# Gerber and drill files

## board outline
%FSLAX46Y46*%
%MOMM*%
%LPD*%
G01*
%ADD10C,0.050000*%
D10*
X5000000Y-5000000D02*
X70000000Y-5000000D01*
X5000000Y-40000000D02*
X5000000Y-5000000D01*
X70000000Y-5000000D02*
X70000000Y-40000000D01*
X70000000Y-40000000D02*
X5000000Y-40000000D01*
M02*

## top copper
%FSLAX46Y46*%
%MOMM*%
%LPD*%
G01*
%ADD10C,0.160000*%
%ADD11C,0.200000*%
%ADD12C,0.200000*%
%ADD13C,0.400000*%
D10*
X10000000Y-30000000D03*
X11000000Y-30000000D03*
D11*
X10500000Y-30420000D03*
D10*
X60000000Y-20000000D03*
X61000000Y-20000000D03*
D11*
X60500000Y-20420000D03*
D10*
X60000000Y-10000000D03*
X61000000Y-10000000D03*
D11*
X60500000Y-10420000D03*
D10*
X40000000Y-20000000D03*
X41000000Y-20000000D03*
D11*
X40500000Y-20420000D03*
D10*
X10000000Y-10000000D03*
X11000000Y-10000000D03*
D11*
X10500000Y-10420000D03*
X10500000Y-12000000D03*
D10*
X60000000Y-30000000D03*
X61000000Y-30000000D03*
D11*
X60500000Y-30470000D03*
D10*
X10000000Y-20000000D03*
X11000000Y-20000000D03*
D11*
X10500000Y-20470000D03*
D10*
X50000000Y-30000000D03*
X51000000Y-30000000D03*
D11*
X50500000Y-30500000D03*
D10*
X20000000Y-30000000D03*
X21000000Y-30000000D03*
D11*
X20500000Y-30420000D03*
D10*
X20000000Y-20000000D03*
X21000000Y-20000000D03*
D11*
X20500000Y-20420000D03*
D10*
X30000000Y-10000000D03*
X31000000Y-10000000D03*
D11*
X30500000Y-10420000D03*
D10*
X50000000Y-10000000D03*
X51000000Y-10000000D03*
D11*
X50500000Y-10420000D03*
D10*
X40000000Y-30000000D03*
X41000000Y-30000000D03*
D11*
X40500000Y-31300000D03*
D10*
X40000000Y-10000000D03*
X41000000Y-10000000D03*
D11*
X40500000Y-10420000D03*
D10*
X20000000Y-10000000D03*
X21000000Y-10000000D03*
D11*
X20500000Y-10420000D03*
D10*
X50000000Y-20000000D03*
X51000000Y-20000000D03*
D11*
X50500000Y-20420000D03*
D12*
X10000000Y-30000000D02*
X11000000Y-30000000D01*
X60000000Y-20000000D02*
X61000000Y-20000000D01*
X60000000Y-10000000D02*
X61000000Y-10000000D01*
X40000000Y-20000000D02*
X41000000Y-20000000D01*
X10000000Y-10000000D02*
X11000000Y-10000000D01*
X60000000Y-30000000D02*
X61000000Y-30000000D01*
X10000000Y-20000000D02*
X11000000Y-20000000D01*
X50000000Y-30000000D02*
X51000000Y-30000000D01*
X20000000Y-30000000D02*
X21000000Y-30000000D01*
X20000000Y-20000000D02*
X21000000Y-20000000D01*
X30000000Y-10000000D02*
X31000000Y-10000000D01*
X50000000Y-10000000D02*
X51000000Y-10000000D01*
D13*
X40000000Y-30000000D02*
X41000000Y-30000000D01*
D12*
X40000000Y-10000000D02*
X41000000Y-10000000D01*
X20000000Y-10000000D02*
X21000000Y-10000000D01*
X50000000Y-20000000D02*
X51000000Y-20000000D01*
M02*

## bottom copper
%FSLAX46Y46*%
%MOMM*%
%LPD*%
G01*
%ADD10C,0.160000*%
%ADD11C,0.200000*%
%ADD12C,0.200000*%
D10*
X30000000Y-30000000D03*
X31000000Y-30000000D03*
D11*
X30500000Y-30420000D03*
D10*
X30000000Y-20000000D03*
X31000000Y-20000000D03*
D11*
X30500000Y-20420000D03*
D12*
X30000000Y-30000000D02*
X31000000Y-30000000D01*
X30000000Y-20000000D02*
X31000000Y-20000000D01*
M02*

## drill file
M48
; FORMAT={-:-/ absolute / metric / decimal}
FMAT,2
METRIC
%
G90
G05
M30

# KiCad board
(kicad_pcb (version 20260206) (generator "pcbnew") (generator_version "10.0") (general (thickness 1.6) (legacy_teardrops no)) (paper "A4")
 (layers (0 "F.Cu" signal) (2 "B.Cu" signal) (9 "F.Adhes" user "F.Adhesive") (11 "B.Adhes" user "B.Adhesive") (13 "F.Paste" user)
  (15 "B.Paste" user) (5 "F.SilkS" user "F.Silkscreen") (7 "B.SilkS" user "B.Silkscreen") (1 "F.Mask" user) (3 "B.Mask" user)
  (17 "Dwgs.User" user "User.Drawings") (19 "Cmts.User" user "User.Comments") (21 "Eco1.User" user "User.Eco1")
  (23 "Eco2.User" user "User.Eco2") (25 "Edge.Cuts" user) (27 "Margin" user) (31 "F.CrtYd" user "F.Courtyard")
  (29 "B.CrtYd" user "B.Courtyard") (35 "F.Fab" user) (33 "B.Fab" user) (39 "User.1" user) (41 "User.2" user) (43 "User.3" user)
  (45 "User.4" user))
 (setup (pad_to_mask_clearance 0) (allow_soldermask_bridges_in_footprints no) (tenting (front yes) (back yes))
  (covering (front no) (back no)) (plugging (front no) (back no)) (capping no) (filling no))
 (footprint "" (layer "F.Cu") (at 10 30)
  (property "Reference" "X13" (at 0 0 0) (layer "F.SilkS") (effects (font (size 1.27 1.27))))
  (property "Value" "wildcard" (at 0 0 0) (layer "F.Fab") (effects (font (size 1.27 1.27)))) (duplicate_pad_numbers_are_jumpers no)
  (pad "1" smd circle (at 0 0) (size 0.16 0.16) (layers "F.Cu") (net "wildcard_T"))
  (pad "2" smd circle (at 1 0) (size 0.16 0.16) (layers "F.Cu") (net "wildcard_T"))
  (pad "3" smd circle (at 0.5 0.42) (size 0.2 0.2) (layers "F.Cu") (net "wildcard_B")))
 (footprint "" (layer "F.Cu") (at 60 20)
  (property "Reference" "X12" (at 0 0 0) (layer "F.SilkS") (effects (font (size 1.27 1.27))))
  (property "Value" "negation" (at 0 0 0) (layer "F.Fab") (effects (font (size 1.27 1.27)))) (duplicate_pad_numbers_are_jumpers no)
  (pad "1" smd circle (at 0 0) (size 0.16 0.16) (layers "F.Cu") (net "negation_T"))
  (pad "2" smd circle (at 1 0) (size 0.16 0.16) (layers "F.Cu") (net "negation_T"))
  (pad "3" smd circle (at 0.5 0.42) (size 0.2 0.2) (layers "F.Cu") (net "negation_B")))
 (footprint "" (layer "F.Cu") (at 60 10)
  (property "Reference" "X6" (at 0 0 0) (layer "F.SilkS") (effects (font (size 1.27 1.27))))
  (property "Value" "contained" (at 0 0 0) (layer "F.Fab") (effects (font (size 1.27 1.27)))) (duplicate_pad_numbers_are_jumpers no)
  (pad "1" smd circle (at 0 0) (size 0.16 0.16) (layers "F.Cu") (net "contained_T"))
  (pad "2" smd circle (at 1 0) (size 0.16 0.16) (layers "F.Cu") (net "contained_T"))
  (pad "3" smd circle (at 0.5 0.42) (size 0.2 0.2) (layers "F.Cu") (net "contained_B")))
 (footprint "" (layer "F.Cu") (at 40 20)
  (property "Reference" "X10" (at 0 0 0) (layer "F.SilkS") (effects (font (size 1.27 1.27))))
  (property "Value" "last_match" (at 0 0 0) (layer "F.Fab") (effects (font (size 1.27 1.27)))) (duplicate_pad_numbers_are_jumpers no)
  (pad "1" smd circle (at 0 0) (size 0.16 0.16) (layers "F.Cu") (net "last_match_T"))
  (pad "2" smd circle (at 1 0) (size 0.16 0.16) (layers "F.Cu") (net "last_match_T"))
  (pad "3" smd circle (at 0.5 0.42) (size 0.2 0.2) (layers "F.Cu") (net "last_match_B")))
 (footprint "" (layer "F.Cu") (at 10 10)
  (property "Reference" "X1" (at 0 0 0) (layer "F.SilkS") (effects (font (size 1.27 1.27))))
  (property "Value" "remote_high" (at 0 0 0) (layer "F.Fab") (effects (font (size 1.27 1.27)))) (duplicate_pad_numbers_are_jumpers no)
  (pad "1" smd circle (at 0 0) (size 0.16 0.16) (layers "F.Cu") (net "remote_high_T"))
  (pad "2" smd circle (at 1 0) (size 0.16 0.16) (layers "F.Cu") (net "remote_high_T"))
  (pad "3" smd circle (at 0.5 0.42) (size 0.2 0.2) (layers "F.Cu") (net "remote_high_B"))
  (pad "4" smd circle (at 0.5 2) (size 0.2 0.2) (layers "F.Cu") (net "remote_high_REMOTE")))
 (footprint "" (layer "F.Cu") (at 60 30)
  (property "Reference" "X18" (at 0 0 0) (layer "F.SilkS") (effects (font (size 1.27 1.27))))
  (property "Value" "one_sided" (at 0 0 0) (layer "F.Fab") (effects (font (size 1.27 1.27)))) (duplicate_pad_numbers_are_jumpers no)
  (pad "1" smd circle (at 0 0) (size 0.16 0.16) (layers "F.Cu") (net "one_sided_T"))
  (pad "2" smd circle (at 1 0) (size 0.16 0.16) (layers "F.Cu") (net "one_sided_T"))
  (pad "3" smd circle (at 0.5 0.47) (size 0.2 0.2) (layers "F.Cu") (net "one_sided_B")))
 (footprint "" (layer "F.Cu") (at 10 20)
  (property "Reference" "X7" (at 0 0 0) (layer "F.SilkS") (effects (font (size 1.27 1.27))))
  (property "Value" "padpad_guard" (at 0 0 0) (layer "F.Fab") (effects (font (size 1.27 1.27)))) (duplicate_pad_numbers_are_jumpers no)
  (pad "1" smd circle (at 0 0) (size 0.16 0.16) (layers "F.Cu") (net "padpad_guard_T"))
  (pad "2" smd circle (at 1 0) (size 0.16 0.16) (layers "F.Cu") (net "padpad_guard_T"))
  (pad "3" smd circle (at 0.5 0.47) (size 0.2 0.2) (layers "F.Cu") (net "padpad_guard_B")))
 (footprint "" (layer "F.Cu") (at 50 30)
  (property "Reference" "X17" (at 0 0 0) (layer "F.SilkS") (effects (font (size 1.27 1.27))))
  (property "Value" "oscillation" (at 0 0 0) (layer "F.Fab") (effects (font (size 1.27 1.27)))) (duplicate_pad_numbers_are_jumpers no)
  (pad "1" smd circle (at 0 0) (size 0.16 0.16) (layers "F.Cu") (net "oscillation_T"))
  (pad "2" smd circle (at 1 0) (size 0.16 0.16) (layers "F.Cu") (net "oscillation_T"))
  (pad "3" smd circle (at 0.5 0.5) (size 0.2 0.2) (layers "F.Cu") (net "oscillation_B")))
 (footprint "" (layer "F.Cu") (at 20 30)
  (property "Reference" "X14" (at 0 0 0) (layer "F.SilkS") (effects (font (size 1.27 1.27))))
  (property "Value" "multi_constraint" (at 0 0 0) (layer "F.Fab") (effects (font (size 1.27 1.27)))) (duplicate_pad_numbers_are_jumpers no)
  (pad "1" smd circle (at 0 0) (size 0.16 0.16) (layers "F.Cu") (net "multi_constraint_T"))
  (pad "2" smd circle (at 1 0) (size 0.16 0.16) (layers "F.Cu") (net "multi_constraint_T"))
  (pad "3" smd circle (at 0.5 0.42) (size 0.2 0.2) (layers "F.Cu") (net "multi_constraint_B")))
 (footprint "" (layer "F.Cu") (at 30 30)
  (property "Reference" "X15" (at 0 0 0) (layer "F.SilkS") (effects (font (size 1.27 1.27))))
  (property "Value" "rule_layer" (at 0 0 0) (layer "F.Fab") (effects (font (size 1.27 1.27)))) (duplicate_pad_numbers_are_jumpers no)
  (pad "1" smd circle (at 0 0) (size 0.16 0.16) (layers "B.Cu") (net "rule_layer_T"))
  (pad "2" smd circle (at 1 0) (size 0.16 0.16) (layers "B.Cu") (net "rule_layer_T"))
  (pad "3" smd circle (at 0.5 0.42) (size 0.2 0.2) (layers "B.Cu") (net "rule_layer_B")))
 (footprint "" (layer "F.Cu") (at 20 20)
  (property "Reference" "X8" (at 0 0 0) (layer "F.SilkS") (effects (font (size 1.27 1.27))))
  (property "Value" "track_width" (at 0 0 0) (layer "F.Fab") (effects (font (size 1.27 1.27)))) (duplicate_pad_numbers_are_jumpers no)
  (pad "1" smd circle (at 0 0) (size 0.16 0.16) (layers "F.Cu") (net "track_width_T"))
  (pad "2" smd circle (at 1 0) (size 0.16 0.16) (layers "F.Cu") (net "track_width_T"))
  (pad "3" smd circle (at 0.5 0.42) (size 0.2 0.2) (layers "F.Cu") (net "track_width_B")))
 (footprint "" (layer "F.Cu") (at 30 10)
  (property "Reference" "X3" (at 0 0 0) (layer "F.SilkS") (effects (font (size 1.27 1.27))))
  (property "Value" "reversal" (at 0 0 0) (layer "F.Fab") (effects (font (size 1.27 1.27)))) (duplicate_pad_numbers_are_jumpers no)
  (pad "1" smd circle (at 0 0) (size 0.16 0.16) (layers "F.Cu") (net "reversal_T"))
  (pad "2" smd circle (at 1 0) (size 0.16 0.16) (layers "F.Cu") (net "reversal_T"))
  (pad "3" smd circle (at 0.5 0.42) (size 0.2 0.2) (layers "F.Cu") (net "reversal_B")))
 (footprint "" (layer "F.Cu") (at 50 10)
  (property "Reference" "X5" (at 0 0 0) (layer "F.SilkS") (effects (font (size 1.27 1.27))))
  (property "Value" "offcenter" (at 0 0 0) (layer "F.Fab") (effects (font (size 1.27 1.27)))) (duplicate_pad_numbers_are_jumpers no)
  (pad "1" smd circle (at 0 0) (size 0.16 0.16) (layers "F.Cu") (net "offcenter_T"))
  (pad "2" smd circle (at 1 0) (size 0.16 0.16) (layers "F.Cu") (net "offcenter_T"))
  (pad "3" smd circle (at 0.5 0.42) (size 0.2 0.2) (layers "F.Cu") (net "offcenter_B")))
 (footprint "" (layer "F.Cu") (at 40 30)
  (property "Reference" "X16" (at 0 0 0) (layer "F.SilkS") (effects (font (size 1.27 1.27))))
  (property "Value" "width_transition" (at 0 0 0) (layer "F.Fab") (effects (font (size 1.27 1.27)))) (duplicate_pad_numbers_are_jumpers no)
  (pad "1" smd circle (at 0 0) (size 0.16 0.16) (layers "F.Cu") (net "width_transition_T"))
  (pad "2" smd circle (at 1 0) (size 0.16 0.16) (layers "F.Cu") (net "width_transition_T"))
  (pad "3" smd circle (at 0.5 1.3) (size 0.2 0.2) (layers "F.Cu") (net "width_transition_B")))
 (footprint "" (layer "F.Cu") (at 30 20)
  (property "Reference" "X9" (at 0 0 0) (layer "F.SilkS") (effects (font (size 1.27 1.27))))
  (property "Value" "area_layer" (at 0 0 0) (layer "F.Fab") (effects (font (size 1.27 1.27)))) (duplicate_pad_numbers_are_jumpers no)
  (pad "1" smd circle (at 0 0) (size 0.16 0.16) (layers "B.Cu") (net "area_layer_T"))
  (pad "2" smd circle (at 1 0) (size 0.16 0.16) (layers "B.Cu") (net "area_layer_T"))
  (pad "3" smd circle (at 0.5 0.42) (size 0.2 0.2) (layers "B.Cu") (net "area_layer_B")))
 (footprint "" (layer "F.Cu") (at 40 10)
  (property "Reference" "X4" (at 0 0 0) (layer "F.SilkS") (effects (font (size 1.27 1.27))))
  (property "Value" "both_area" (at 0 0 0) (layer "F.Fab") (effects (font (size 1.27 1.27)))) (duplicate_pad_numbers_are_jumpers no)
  (pad "1" smd circle (at 0 0) (size 0.16 0.16) (layers "F.Cu") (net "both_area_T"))
  (pad "2" smd circle (at 1 0) (size 0.16 0.16) (layers "F.Cu") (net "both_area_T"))
  (pad "3" smd circle (at 0.5 0.42) (size 0.2 0.2) (layers "F.Cu") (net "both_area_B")))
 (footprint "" (layer "F.Cu") (at 20 10)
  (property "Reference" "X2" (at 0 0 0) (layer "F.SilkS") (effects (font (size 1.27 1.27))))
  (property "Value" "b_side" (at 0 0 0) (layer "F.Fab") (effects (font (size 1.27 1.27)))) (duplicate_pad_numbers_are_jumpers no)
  (pad "1" smd circle (at 0 0) (size 0.16 0.16) (layers "F.Cu") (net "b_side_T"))
  (pad "2" smd circle (at 1 0) (size 0.16 0.16) (layers "F.Cu") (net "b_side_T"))
  (pad "3" smd circle (at 0.5 0.42) (size 0.2 0.2) (layers "F.Cu") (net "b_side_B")))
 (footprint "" (layer "F.Cu") (at 50 20)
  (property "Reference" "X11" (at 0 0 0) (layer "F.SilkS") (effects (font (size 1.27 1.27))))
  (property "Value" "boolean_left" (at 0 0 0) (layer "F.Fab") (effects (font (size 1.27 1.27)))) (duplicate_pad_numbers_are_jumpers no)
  (pad "1" smd circle (at 0 0) (size 0.16 0.16) (layers "F.Cu") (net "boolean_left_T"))
  (pad "2" smd circle (at 1 0) (size 0.16 0.16) (layers "F.Cu") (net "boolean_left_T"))
  (pad "3" smd circle (at 0.5 0.42) (size 0.2 0.2) (layers "F.Cu") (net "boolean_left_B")))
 (gr_line (start 5 5) (end 70 5) (stroke (width 0.05) (type default)) (layer "Edge.Cuts"))
 (gr_line (start 5 40) (end 5 5) (stroke (width 0.05) (type default)) (layer "Edge.Cuts"))
 (gr_line (start 70 5) (end 70 40) (stroke (width 0.05) (type default)) (layer "Edge.Cuts"))
 (gr_line (start 70 40) (end 5 40) (stroke (width 0.05) (type default)) (layer "Edge.Cuts"))
 (segment (start 10 30) (end 11 30) (width 0.2) (layer "F.Cu") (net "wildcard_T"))
 (segment (start 60 20) (end 61 20) (width 0.2) (layer "F.Cu") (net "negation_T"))
 (segment (start 60 10) (end 61 10) (width 0.2) (layer "F.Cu") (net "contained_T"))
 (segment (start 40 20) (end 41 20) (width 0.2) (layer "F.Cu") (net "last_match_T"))
 (segment (start 10 10) (end 11 10) (width 0.2) (layer "F.Cu") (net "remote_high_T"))
 (segment (start 60 30) (end 61 30) (width 0.2) (layer "F.Cu") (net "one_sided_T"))
 (segment (start 10 20) (end 11 20) (width 0.2) (layer "F.Cu") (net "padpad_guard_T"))
 (segment (start 50 30) (end 51 30) (width 0.2) (layer "F.Cu") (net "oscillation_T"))
 (segment (start 20 30) (end 21 30) (width 0.2) (layer "F.Cu") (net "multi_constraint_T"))
 (segment (start 30 30) (end 31 30) (width 0.2) (layer "B.Cu") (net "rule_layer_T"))
 (segment (start 20 20) (end 21 20) (width 0.2) (layer "F.Cu") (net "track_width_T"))
 (segment (start 30 10) (end 31 10) (width 0.2) (layer "F.Cu") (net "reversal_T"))
 (segment (start 50 10) (end 51 10) (width 0.2) (layer "F.Cu") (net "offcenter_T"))
 (segment (start 40 30) (end 41 30) (width 0.4) (layer "F.Cu") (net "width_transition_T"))
 (segment (start 30 20) (end 31 20) (width 0.2) (layer "B.Cu") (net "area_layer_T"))
 (segment (start 40 10) (end 41 10) (width 0.2) (layer "F.Cu") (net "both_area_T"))
 (segment (start 20 10) (end 21 10) (width 0.2) (layer "F.Cu") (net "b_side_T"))
 (segment (start 50 20) (end 51 20) (width 0.2) (layer "F.Cu") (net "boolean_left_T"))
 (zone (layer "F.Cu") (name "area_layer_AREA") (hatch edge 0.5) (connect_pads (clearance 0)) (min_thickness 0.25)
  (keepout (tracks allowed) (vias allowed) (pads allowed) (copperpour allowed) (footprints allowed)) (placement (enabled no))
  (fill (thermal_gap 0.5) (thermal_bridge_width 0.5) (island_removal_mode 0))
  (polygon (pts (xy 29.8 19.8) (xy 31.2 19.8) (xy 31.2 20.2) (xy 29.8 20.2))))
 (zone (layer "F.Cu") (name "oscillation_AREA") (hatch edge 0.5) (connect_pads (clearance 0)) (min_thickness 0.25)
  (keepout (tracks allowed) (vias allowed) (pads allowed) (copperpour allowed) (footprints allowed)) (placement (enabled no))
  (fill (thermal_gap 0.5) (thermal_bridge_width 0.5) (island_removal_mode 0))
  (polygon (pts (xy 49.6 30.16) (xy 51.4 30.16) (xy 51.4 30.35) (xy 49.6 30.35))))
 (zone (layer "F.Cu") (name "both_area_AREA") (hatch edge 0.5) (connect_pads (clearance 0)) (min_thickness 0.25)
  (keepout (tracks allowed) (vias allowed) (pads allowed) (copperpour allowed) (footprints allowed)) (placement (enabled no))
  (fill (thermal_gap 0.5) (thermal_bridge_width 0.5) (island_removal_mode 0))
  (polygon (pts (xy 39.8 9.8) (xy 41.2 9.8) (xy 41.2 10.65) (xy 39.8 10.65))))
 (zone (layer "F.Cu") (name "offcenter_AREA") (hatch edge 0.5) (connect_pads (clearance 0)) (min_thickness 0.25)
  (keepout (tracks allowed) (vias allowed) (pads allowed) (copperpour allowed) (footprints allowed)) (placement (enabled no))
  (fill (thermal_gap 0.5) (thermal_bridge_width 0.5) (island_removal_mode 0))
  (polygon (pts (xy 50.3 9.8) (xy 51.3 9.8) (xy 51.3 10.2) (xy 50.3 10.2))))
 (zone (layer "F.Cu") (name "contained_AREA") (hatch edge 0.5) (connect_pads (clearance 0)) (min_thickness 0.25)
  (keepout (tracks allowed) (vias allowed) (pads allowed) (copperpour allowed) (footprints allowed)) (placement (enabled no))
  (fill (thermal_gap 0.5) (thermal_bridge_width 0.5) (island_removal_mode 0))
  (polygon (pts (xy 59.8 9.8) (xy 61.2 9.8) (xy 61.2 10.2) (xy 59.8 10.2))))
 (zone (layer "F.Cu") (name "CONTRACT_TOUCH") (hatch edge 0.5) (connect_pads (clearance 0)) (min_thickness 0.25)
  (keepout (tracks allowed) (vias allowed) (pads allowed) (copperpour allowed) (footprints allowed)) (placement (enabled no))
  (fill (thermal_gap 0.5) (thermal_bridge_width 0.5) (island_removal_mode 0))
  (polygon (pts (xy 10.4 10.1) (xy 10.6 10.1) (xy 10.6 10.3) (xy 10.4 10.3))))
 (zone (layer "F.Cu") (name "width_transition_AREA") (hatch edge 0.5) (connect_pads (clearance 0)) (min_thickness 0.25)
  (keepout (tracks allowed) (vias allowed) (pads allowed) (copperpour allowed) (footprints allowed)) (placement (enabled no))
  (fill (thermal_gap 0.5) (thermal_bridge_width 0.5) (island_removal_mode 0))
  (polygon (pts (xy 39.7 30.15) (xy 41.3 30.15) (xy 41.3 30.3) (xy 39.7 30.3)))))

